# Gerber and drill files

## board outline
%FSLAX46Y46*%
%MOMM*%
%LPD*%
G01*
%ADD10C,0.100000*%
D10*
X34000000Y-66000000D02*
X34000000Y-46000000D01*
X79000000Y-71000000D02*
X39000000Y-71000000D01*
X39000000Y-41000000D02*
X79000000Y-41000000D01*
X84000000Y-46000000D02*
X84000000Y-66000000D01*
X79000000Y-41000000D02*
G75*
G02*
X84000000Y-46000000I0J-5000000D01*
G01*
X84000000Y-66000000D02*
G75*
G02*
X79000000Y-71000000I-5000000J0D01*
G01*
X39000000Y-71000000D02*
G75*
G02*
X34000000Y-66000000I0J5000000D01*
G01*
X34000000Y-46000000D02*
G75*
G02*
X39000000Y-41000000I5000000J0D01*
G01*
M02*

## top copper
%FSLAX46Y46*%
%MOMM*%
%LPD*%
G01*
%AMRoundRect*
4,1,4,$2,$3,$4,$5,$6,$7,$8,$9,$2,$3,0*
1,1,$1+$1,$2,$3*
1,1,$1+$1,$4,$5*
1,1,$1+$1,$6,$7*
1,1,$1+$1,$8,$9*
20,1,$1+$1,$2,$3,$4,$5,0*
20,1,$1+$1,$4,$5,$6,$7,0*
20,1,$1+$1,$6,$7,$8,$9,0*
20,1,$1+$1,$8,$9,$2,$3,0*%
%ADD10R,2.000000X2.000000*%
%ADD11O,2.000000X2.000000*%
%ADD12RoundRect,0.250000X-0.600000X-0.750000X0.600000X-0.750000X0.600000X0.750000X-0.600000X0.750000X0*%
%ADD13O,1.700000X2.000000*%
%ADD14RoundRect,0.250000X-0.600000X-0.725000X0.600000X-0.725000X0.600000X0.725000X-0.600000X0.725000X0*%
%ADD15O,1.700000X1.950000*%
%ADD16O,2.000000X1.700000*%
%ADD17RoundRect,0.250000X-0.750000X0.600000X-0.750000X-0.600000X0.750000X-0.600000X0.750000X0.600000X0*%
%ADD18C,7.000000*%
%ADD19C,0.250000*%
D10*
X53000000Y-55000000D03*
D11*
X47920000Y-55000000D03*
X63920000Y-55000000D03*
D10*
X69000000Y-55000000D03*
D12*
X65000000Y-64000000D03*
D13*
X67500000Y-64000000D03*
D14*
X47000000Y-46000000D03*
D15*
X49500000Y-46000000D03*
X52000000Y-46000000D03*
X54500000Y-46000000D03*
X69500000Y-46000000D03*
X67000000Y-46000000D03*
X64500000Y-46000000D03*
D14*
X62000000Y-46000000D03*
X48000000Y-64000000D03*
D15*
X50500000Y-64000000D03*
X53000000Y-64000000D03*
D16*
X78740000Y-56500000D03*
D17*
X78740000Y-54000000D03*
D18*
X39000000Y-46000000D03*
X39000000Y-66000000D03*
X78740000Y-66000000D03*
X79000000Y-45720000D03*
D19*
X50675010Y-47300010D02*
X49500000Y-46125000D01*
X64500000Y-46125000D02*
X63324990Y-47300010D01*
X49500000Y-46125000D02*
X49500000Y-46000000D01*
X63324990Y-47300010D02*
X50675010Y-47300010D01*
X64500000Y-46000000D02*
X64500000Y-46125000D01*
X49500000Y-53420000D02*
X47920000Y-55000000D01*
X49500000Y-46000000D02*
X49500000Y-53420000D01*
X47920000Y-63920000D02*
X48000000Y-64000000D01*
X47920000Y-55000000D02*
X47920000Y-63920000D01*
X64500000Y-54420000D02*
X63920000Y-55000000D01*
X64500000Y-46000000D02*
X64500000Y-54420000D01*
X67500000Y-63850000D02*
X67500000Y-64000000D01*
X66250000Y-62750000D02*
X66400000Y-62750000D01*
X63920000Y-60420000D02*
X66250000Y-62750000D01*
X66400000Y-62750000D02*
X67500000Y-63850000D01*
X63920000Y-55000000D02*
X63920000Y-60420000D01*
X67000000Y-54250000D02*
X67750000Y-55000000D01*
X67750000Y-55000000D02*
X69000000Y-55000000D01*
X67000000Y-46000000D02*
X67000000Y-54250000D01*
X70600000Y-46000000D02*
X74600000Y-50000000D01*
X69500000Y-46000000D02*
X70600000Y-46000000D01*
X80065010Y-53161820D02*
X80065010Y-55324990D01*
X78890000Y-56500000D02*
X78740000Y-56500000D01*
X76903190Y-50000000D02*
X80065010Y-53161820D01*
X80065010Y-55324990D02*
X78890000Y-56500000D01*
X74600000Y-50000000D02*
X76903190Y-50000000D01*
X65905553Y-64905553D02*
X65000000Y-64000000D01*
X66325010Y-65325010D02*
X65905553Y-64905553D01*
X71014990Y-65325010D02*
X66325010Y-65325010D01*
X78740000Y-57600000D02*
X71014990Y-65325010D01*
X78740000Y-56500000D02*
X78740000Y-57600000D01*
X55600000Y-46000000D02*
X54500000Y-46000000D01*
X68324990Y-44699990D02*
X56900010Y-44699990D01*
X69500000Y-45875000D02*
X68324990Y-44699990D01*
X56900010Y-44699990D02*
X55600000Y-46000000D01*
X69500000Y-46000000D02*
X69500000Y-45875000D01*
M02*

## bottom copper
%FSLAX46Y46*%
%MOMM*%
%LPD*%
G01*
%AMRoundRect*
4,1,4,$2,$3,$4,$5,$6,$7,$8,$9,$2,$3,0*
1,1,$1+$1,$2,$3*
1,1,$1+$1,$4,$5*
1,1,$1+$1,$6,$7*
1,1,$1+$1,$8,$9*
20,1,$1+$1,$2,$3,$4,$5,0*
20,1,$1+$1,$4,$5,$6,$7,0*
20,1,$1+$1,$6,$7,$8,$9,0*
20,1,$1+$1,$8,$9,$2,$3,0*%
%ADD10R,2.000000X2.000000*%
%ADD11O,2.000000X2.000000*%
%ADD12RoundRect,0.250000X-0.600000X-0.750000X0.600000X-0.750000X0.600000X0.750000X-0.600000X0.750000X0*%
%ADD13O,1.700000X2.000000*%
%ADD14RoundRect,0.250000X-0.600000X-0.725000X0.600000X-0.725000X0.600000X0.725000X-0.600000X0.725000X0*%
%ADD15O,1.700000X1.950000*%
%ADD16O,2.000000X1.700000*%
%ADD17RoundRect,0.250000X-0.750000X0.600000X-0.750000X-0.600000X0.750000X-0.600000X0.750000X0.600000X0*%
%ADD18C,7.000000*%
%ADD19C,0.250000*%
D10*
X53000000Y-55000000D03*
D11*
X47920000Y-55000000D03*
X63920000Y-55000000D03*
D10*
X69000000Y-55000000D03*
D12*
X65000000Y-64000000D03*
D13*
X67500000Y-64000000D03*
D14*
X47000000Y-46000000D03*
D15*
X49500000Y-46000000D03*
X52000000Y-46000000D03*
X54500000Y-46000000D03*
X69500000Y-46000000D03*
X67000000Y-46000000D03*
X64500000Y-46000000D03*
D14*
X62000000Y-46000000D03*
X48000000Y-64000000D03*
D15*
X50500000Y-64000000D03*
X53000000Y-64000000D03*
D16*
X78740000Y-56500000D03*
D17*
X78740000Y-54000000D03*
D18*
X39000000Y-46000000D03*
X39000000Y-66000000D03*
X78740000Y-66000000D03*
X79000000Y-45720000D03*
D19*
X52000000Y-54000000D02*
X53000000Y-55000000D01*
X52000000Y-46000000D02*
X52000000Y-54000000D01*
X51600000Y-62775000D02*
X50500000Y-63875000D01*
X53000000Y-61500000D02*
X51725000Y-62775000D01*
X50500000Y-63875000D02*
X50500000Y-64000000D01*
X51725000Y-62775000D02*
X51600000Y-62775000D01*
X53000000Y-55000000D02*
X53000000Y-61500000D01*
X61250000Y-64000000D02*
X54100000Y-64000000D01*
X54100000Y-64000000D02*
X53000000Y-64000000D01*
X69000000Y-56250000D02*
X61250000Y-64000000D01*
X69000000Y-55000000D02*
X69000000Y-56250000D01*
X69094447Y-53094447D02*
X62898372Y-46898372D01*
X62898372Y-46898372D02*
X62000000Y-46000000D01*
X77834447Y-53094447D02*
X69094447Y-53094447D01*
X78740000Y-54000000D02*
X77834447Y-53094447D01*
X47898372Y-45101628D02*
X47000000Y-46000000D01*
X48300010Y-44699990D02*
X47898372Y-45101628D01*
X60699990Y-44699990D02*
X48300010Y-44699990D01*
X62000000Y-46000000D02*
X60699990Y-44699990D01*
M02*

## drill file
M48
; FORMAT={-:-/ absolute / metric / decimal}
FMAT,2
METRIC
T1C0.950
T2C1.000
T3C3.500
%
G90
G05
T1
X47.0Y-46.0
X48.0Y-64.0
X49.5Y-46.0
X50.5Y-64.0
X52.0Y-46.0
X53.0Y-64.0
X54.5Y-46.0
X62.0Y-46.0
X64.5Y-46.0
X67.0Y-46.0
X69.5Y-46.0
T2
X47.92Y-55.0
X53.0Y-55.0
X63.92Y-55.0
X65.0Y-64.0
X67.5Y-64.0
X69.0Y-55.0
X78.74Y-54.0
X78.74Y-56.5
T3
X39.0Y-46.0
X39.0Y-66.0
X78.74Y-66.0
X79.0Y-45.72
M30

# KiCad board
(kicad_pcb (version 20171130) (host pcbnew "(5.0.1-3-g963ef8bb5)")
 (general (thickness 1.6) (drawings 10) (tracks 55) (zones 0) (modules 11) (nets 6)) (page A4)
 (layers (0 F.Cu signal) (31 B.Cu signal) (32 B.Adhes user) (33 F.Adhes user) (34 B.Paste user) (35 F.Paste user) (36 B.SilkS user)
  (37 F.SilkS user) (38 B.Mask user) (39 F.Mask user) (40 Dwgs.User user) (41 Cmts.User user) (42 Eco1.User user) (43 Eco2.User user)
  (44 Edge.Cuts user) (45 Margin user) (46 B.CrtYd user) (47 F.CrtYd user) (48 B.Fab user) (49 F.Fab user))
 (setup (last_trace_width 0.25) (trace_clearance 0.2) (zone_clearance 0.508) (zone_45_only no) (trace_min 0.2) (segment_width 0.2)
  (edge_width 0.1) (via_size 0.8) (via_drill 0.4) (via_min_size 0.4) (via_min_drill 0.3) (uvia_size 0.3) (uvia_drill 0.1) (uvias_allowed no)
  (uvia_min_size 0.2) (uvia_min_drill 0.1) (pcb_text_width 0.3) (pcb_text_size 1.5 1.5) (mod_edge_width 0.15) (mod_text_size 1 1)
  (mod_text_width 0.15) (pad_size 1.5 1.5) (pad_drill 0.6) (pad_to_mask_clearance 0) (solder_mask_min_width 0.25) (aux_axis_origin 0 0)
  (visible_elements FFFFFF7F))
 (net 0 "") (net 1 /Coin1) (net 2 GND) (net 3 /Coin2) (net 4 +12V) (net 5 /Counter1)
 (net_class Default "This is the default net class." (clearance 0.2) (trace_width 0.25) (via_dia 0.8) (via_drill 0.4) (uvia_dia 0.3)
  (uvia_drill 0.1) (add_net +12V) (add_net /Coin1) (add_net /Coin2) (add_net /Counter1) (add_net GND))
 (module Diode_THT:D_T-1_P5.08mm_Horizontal (layer F.Cu) (at 53 55 180)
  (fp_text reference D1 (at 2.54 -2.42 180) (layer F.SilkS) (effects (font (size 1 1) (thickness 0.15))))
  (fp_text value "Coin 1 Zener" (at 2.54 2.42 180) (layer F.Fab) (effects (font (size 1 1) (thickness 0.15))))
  (pad 1 thru_hole rect (at 0 0 180) (size 2 2) (drill 1) (layers *.Cu *.Mask) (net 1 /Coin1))
  (pad 2 thru_hole oval (at 5.08 0 180) (size 2 2) (drill 1) (layers *.Cu *.Mask) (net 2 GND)))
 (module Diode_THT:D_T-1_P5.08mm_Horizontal (layer F.Cu) (at 69 55 180)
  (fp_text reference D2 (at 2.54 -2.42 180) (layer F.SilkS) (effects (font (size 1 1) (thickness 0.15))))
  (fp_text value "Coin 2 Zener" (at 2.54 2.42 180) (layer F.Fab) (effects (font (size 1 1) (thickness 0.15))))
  (pad 2 thru_hole oval (at 5.08 0 180) (size 2 2) (drill 1) (layers *.Cu *.Mask) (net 2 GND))
  (pad 1 thru_hole rect (at 0 0 180) (size 2 2) (drill 1) (layers *.Cu *.Mask) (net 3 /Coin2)))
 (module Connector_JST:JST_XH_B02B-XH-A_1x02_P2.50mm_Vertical (layer F.Cu) (at 65 64)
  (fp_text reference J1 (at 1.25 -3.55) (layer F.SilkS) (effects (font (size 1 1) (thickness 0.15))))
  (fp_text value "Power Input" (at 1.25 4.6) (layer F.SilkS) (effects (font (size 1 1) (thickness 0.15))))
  (pad 1 thru_hole roundrect (at 0 0) (size 1.7 2) (drill 1) (layers *.Cu *.Mask) (roundrect_rratio 0.147059) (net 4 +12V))
  (pad 2 thru_hole oval (at 2.5 0) (size 1.7 2) (drill 1) (layers *.Cu *.Mask) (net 2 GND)))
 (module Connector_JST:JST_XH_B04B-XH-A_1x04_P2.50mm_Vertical (layer F.Cu) (at 47 46)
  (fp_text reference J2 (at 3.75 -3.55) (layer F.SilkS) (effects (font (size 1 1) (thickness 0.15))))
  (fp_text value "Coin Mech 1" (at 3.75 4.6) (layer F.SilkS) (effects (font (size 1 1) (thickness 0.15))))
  (pad 1 thru_hole roundrect (at 0 0) (size 1.7 1.95) (drill 0.95) (layers *.Cu *.Mask) (roundrect_rratio 0.147059) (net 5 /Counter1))
  (pad 2 thru_hole oval (at 2.5 0) (size 1.7 1.95) (drill 0.95) (layers *.Cu *.Mask) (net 2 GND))
  (pad 3 thru_hole oval (at 5 0) (size 1.7 1.95) (drill 0.95) (layers *.Cu *.Mask) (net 1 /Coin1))
  (pad 4 thru_hole oval (at 7.5 0) (size 1.7 1.95) (drill 0.95) (layers *.Cu *.Mask) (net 4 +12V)))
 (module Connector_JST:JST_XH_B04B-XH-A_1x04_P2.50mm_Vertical (layer F.Cu) (at 62 46)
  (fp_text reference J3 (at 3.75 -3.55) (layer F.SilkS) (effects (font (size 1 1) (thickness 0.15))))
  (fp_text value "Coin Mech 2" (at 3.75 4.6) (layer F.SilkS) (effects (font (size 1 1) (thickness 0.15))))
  (pad 4 thru_hole oval (at 7.5 0) (size 1.7 1.95) (drill 0.95) (layers *.Cu *.Mask) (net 4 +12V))
  (pad 3 thru_hole oval (at 5 0) (size 1.7 1.95) (drill 0.95) (layers *.Cu *.Mask) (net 3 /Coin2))
  (pad 2 thru_hole oval (at 2.5 0) (size 1.7 1.95) (drill 0.95) (layers *.Cu *.Mask) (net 2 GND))
  (pad 1 thru_hole roundrect (at 0 0) (size 1.7 1.95) (drill 0.95) (layers *.Cu *.Mask) (roundrect_rratio 0.147059) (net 5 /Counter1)))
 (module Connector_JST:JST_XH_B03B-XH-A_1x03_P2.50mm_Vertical (layer F.Cu) (at 48 64)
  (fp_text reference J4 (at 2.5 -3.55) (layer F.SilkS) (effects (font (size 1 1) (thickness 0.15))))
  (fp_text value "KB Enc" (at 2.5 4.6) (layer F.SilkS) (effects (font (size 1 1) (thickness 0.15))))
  (pad 1 thru_hole roundrect (at 0 0) (size 1.7 1.95) (drill 0.95) (layers *.Cu *.Mask) (roundrect_rratio 0.147059) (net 2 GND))
  (pad 2 thru_hole oval (at 2.5 0) (size 1.7 1.95) (drill 0.95) (layers *.Cu *.Mask) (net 1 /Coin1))
  (pad 3 thru_hole oval (at 5 0) (size 1.7 1.95) (drill 0.95) (layers *.Cu *.Mask) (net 3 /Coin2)))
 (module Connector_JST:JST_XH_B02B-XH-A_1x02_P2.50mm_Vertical (layer F.Cu) (at 78.74 54 270)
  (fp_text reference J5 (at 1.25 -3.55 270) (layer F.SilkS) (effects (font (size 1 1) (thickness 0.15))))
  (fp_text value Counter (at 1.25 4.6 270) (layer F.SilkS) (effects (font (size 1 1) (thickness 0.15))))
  (pad 2 thru_hole oval (at 2.5 0 270) (size 1.7 2) (drill 1) (layers *.Cu *.Mask) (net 4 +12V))
  (pad 1 thru_hole roundrect (at 0 0 270) (size 1.7 2) (drill 1) (layers *.Cu *.Mask) (roundrect_rratio 0.147059) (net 5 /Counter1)))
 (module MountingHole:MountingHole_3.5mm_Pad (layer F.Cu) (at 39 46)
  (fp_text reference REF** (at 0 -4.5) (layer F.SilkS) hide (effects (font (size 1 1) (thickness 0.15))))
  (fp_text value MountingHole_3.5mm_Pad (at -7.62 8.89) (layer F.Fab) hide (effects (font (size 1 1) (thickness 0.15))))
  (pad 1 thru_hole circle (at 0 0) (size 7 7) (drill 3.5) (layers *.Cu *.Mask)))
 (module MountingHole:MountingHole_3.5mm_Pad (layer F.Cu) (at 39 66)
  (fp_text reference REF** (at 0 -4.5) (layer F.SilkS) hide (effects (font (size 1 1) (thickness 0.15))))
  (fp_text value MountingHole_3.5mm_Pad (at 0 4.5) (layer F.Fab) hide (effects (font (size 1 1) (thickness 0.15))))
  (pad 1 thru_hole circle (at 0 0) (size 7 7) (drill 3.5) (layers *.Cu *.Mask)))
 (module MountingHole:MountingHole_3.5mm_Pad (layer F.Cu) (at 78.74 66)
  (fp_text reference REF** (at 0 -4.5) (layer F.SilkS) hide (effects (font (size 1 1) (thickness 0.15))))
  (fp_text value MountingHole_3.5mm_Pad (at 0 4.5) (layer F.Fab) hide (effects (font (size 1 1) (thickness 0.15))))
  (pad 1 thru_hole circle (at 0 0) (size 7 7) (drill 3.5) (layers *.Cu *.Mask)))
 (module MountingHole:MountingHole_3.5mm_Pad (layer F.Cu) (at 79 45.72)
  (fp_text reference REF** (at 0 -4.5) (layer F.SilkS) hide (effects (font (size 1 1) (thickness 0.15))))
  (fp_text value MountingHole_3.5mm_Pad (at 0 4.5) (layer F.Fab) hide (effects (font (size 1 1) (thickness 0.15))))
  (pad 1 thru_hole circle (at 0 0) (size 7 7) (drill 3.5) (layers *.Cu *.Mask)))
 (gr_line (start 34 66) (end 34 46) (layer Edge.Cuts) (width 0.1))
 (gr_line (start 79 71) (end 39 71) (layer Edge.Cuts) (width 0.1))
 (gr_line (start 39 41) (end 79 41) (layer Edge.Cuts) (width 0.1))
 (gr_line (start 84 46) (end 84 66) (layer Edge.Cuts) (width 0.1))
 (gr_arc (start 79 46) (end 84 46) (angle -90) (layer Edge.Cuts) (width 0.1))
 (gr_arc (start 79 66) (end 79 71) (angle -90) (layer Edge.Cuts) (width 0.1))
 (gr_arc (start 39 66) (end 34 66) (angle -90) (layer Edge.Cuts) (width 0.1))
 (gr_arc (start 39 46) (end 39 41) (angle -90) (layer Edge.Cuts) (width 0.1))
 (segment (start 52 54) (end 53 55) (width 0.25) (layer B.Cu) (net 1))
 (segment (start 52 46) (end 52 54) (width 0.25) (layer B.Cu) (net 1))
 (segment (start 51.6 62.775) (end 50.5 63.875) (width 0.25) (layer B.Cu) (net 1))
 (segment (start 53 61.5) (end 51.725 62.775) (width 0.25) (layer B.Cu) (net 1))
 (segment (start 50.5 63.875) (end 50.5 64) (width 0.25) (layer B.Cu) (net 1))
 (segment (start 51.725 62.775) (end 51.6 62.775) (width 0.25) (layer B.Cu) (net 1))
 (segment (start 53 55) (end 53 61.5) (width 0.25) (layer B.Cu) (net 1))
 (segment (start 50.67501 47.30001) (end 49.5 46.125) (width 0.25) (layer F.Cu) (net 2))
 (segment (start 64.5 46.125) (end 63.32499 47.30001) (width 0.25) (layer F.Cu) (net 2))
 (segment (start 49.5 46.125) (end 49.5 46) (width 0.25) (layer F.Cu) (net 2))
 (segment (start 63.32499 47.30001) (end 50.67501 47.30001) (width 0.25) (layer F.Cu) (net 2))
 (segment (start 64.5 46) (end 64.5 46.125) (width 0.25) (layer F.Cu) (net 2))
 (segment (start 49.5 53.42) (end 47.92 55) (width 0.25) (layer F.Cu) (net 2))
 (segment (start 49.5 46) (end 49.5 53.42) (width 0.25) (layer F.Cu) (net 2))
 (segment (start 47.92 63.92) (end 48 64) (width 0.25) (layer F.Cu) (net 2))
 (segment (start 47.92 55) (end 47.92 63.92) (width 0.25) (layer F.Cu) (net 2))
 (segment (start 64.5 54.42) (end 63.92 55) (width 0.25) (layer F.Cu) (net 2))
 (segment (start 64.5 46) (end 64.5 54.42) (width 0.25) (layer F.Cu) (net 2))
 (segment (start 67.5 63.85) (end 67.5 64) (width 0.25) (layer F.Cu) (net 2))
 (segment (start 66.25 62.75) (end 66.4 62.75) (width 0.25) (layer F.Cu) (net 2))
 (segment (start 63.92 60.42) (end 66.25 62.75) (width 0.25) (layer F.Cu) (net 2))
 (segment (start 66.4 62.75) (end 67.5 63.85) (width 0.25) (layer F.Cu) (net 2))
 (segment (start 63.92 55) (end 63.92 60.42) (width 0.25) (layer F.Cu) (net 2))
 (segment (start 61.25 64) (end 54.1 64) (width 0.25) (layer B.Cu) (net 3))
 (segment (start 54.1 64) (end 53 64) (width 0.25) (layer B.Cu) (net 3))
 (segment (start 69 56.25) (end 61.25 64) (width 0.25) (layer B.Cu) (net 3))
 (segment (start 69 55) (end 69 56.25) (width 0.25) (layer B.Cu) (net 3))
 (segment (start 67 54.25) (end 67.75 55) (width 0.25) (layer F.Cu) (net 3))
 (segment (start 67.75 55) (end 69 55) (width 0.25) (layer F.Cu) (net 3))
 (segment (start 67 46) (end 67 54.25) (width 0.25) (layer F.Cu) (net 3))
 (segment (start 70.6 46) (end 74.6 50) (width 0.25) (layer F.Cu) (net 4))
 (segment (start 69.5 46) (end 70.6 46) (width 0.25) (layer F.Cu) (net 4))
 (segment (start 80.06501 53.16182) (end 80.06501 55.32499) (width 0.25) (layer F.Cu) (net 4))
 (segment (start 78.89 56.5) (end 78.74 56.5) (width 0.25) (layer F.Cu) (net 4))
 (segment (start 76.90319 50) (end 80.06501 53.16182) (width 0.25) (layer F.Cu) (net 4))
 (segment (start 80.06501 55.32499) (end 78.89 56.5) (width 0.25) (layer F.Cu) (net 4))
 (segment (start 74.6 50) (end 76.90319 50) (width 0.25) (layer F.Cu) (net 4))
 (segment (start 65.905553 64.905553) (end 65 64) (width 0.25) (layer F.Cu) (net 4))
 (segment (start 66.32501 65.32501) (end 65.905553 64.905553) (width 0.25) (layer F.Cu) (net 4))
 (segment (start 71.01499 65.32501) (end 66.32501 65.32501) (width 0.25) (layer F.Cu) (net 4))
 (segment (start 78.74 57.6) (end 71.01499 65.32501) (width 0.25) (layer F.Cu) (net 4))
 (segment (start 78.74 56.5) (end 78.74 57.6) (width 0.25) (layer F.Cu) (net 4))
 (segment (start 55.6 46) (end 54.5 46) (width 0.25) (layer F.Cu) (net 4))
 (segment (start 68.32499 44.69999) (end 56.90001 44.69999) (width 0.25) (layer F.Cu) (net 4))
 (segment (start 69.5 45.875) (end 68.32499 44.69999) (width 0.25) (layer F.Cu) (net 4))
 (segment (start 56.90001 44.69999) (end 55.6 46) (width 0.25) (layer F.Cu) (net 4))
 (segment (start 69.5 46) (end 69.5 45.875) (width 0.25) (layer F.Cu) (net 4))
 (segment (start 69.094447 53.094447) (end 62.898372 46.898372) (width 0.25) (layer B.Cu) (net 5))
 (segment (start 62.898372 46.898372) (end 62 46) (width 0.25) (layer B.Cu) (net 5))
 (segment (start 77.834447 53.094447) (end 69.094447 53.094447) (width 0.25) (layer B.Cu) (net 5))
 (segment (start 78.74 54) (end 77.834447 53.094447) (width 0.25) (layer B.Cu) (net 5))
 (segment (start 47.898372 45.101628) (end 47 46) (width 0.25) (layer B.Cu) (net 5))
 (segment (start 48.30001 44.69999) (end 47.898372 45.101628) (width 0.25) (layer B.Cu) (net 5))
 (segment (start 60.69999 44.69999) (end 48.30001 44.69999) (width 0.25) (layer B.Cu) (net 5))
 (segment (start 62 46) (end 60.69999 44.69999) (width 0.25) (layer B.Cu) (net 5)))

